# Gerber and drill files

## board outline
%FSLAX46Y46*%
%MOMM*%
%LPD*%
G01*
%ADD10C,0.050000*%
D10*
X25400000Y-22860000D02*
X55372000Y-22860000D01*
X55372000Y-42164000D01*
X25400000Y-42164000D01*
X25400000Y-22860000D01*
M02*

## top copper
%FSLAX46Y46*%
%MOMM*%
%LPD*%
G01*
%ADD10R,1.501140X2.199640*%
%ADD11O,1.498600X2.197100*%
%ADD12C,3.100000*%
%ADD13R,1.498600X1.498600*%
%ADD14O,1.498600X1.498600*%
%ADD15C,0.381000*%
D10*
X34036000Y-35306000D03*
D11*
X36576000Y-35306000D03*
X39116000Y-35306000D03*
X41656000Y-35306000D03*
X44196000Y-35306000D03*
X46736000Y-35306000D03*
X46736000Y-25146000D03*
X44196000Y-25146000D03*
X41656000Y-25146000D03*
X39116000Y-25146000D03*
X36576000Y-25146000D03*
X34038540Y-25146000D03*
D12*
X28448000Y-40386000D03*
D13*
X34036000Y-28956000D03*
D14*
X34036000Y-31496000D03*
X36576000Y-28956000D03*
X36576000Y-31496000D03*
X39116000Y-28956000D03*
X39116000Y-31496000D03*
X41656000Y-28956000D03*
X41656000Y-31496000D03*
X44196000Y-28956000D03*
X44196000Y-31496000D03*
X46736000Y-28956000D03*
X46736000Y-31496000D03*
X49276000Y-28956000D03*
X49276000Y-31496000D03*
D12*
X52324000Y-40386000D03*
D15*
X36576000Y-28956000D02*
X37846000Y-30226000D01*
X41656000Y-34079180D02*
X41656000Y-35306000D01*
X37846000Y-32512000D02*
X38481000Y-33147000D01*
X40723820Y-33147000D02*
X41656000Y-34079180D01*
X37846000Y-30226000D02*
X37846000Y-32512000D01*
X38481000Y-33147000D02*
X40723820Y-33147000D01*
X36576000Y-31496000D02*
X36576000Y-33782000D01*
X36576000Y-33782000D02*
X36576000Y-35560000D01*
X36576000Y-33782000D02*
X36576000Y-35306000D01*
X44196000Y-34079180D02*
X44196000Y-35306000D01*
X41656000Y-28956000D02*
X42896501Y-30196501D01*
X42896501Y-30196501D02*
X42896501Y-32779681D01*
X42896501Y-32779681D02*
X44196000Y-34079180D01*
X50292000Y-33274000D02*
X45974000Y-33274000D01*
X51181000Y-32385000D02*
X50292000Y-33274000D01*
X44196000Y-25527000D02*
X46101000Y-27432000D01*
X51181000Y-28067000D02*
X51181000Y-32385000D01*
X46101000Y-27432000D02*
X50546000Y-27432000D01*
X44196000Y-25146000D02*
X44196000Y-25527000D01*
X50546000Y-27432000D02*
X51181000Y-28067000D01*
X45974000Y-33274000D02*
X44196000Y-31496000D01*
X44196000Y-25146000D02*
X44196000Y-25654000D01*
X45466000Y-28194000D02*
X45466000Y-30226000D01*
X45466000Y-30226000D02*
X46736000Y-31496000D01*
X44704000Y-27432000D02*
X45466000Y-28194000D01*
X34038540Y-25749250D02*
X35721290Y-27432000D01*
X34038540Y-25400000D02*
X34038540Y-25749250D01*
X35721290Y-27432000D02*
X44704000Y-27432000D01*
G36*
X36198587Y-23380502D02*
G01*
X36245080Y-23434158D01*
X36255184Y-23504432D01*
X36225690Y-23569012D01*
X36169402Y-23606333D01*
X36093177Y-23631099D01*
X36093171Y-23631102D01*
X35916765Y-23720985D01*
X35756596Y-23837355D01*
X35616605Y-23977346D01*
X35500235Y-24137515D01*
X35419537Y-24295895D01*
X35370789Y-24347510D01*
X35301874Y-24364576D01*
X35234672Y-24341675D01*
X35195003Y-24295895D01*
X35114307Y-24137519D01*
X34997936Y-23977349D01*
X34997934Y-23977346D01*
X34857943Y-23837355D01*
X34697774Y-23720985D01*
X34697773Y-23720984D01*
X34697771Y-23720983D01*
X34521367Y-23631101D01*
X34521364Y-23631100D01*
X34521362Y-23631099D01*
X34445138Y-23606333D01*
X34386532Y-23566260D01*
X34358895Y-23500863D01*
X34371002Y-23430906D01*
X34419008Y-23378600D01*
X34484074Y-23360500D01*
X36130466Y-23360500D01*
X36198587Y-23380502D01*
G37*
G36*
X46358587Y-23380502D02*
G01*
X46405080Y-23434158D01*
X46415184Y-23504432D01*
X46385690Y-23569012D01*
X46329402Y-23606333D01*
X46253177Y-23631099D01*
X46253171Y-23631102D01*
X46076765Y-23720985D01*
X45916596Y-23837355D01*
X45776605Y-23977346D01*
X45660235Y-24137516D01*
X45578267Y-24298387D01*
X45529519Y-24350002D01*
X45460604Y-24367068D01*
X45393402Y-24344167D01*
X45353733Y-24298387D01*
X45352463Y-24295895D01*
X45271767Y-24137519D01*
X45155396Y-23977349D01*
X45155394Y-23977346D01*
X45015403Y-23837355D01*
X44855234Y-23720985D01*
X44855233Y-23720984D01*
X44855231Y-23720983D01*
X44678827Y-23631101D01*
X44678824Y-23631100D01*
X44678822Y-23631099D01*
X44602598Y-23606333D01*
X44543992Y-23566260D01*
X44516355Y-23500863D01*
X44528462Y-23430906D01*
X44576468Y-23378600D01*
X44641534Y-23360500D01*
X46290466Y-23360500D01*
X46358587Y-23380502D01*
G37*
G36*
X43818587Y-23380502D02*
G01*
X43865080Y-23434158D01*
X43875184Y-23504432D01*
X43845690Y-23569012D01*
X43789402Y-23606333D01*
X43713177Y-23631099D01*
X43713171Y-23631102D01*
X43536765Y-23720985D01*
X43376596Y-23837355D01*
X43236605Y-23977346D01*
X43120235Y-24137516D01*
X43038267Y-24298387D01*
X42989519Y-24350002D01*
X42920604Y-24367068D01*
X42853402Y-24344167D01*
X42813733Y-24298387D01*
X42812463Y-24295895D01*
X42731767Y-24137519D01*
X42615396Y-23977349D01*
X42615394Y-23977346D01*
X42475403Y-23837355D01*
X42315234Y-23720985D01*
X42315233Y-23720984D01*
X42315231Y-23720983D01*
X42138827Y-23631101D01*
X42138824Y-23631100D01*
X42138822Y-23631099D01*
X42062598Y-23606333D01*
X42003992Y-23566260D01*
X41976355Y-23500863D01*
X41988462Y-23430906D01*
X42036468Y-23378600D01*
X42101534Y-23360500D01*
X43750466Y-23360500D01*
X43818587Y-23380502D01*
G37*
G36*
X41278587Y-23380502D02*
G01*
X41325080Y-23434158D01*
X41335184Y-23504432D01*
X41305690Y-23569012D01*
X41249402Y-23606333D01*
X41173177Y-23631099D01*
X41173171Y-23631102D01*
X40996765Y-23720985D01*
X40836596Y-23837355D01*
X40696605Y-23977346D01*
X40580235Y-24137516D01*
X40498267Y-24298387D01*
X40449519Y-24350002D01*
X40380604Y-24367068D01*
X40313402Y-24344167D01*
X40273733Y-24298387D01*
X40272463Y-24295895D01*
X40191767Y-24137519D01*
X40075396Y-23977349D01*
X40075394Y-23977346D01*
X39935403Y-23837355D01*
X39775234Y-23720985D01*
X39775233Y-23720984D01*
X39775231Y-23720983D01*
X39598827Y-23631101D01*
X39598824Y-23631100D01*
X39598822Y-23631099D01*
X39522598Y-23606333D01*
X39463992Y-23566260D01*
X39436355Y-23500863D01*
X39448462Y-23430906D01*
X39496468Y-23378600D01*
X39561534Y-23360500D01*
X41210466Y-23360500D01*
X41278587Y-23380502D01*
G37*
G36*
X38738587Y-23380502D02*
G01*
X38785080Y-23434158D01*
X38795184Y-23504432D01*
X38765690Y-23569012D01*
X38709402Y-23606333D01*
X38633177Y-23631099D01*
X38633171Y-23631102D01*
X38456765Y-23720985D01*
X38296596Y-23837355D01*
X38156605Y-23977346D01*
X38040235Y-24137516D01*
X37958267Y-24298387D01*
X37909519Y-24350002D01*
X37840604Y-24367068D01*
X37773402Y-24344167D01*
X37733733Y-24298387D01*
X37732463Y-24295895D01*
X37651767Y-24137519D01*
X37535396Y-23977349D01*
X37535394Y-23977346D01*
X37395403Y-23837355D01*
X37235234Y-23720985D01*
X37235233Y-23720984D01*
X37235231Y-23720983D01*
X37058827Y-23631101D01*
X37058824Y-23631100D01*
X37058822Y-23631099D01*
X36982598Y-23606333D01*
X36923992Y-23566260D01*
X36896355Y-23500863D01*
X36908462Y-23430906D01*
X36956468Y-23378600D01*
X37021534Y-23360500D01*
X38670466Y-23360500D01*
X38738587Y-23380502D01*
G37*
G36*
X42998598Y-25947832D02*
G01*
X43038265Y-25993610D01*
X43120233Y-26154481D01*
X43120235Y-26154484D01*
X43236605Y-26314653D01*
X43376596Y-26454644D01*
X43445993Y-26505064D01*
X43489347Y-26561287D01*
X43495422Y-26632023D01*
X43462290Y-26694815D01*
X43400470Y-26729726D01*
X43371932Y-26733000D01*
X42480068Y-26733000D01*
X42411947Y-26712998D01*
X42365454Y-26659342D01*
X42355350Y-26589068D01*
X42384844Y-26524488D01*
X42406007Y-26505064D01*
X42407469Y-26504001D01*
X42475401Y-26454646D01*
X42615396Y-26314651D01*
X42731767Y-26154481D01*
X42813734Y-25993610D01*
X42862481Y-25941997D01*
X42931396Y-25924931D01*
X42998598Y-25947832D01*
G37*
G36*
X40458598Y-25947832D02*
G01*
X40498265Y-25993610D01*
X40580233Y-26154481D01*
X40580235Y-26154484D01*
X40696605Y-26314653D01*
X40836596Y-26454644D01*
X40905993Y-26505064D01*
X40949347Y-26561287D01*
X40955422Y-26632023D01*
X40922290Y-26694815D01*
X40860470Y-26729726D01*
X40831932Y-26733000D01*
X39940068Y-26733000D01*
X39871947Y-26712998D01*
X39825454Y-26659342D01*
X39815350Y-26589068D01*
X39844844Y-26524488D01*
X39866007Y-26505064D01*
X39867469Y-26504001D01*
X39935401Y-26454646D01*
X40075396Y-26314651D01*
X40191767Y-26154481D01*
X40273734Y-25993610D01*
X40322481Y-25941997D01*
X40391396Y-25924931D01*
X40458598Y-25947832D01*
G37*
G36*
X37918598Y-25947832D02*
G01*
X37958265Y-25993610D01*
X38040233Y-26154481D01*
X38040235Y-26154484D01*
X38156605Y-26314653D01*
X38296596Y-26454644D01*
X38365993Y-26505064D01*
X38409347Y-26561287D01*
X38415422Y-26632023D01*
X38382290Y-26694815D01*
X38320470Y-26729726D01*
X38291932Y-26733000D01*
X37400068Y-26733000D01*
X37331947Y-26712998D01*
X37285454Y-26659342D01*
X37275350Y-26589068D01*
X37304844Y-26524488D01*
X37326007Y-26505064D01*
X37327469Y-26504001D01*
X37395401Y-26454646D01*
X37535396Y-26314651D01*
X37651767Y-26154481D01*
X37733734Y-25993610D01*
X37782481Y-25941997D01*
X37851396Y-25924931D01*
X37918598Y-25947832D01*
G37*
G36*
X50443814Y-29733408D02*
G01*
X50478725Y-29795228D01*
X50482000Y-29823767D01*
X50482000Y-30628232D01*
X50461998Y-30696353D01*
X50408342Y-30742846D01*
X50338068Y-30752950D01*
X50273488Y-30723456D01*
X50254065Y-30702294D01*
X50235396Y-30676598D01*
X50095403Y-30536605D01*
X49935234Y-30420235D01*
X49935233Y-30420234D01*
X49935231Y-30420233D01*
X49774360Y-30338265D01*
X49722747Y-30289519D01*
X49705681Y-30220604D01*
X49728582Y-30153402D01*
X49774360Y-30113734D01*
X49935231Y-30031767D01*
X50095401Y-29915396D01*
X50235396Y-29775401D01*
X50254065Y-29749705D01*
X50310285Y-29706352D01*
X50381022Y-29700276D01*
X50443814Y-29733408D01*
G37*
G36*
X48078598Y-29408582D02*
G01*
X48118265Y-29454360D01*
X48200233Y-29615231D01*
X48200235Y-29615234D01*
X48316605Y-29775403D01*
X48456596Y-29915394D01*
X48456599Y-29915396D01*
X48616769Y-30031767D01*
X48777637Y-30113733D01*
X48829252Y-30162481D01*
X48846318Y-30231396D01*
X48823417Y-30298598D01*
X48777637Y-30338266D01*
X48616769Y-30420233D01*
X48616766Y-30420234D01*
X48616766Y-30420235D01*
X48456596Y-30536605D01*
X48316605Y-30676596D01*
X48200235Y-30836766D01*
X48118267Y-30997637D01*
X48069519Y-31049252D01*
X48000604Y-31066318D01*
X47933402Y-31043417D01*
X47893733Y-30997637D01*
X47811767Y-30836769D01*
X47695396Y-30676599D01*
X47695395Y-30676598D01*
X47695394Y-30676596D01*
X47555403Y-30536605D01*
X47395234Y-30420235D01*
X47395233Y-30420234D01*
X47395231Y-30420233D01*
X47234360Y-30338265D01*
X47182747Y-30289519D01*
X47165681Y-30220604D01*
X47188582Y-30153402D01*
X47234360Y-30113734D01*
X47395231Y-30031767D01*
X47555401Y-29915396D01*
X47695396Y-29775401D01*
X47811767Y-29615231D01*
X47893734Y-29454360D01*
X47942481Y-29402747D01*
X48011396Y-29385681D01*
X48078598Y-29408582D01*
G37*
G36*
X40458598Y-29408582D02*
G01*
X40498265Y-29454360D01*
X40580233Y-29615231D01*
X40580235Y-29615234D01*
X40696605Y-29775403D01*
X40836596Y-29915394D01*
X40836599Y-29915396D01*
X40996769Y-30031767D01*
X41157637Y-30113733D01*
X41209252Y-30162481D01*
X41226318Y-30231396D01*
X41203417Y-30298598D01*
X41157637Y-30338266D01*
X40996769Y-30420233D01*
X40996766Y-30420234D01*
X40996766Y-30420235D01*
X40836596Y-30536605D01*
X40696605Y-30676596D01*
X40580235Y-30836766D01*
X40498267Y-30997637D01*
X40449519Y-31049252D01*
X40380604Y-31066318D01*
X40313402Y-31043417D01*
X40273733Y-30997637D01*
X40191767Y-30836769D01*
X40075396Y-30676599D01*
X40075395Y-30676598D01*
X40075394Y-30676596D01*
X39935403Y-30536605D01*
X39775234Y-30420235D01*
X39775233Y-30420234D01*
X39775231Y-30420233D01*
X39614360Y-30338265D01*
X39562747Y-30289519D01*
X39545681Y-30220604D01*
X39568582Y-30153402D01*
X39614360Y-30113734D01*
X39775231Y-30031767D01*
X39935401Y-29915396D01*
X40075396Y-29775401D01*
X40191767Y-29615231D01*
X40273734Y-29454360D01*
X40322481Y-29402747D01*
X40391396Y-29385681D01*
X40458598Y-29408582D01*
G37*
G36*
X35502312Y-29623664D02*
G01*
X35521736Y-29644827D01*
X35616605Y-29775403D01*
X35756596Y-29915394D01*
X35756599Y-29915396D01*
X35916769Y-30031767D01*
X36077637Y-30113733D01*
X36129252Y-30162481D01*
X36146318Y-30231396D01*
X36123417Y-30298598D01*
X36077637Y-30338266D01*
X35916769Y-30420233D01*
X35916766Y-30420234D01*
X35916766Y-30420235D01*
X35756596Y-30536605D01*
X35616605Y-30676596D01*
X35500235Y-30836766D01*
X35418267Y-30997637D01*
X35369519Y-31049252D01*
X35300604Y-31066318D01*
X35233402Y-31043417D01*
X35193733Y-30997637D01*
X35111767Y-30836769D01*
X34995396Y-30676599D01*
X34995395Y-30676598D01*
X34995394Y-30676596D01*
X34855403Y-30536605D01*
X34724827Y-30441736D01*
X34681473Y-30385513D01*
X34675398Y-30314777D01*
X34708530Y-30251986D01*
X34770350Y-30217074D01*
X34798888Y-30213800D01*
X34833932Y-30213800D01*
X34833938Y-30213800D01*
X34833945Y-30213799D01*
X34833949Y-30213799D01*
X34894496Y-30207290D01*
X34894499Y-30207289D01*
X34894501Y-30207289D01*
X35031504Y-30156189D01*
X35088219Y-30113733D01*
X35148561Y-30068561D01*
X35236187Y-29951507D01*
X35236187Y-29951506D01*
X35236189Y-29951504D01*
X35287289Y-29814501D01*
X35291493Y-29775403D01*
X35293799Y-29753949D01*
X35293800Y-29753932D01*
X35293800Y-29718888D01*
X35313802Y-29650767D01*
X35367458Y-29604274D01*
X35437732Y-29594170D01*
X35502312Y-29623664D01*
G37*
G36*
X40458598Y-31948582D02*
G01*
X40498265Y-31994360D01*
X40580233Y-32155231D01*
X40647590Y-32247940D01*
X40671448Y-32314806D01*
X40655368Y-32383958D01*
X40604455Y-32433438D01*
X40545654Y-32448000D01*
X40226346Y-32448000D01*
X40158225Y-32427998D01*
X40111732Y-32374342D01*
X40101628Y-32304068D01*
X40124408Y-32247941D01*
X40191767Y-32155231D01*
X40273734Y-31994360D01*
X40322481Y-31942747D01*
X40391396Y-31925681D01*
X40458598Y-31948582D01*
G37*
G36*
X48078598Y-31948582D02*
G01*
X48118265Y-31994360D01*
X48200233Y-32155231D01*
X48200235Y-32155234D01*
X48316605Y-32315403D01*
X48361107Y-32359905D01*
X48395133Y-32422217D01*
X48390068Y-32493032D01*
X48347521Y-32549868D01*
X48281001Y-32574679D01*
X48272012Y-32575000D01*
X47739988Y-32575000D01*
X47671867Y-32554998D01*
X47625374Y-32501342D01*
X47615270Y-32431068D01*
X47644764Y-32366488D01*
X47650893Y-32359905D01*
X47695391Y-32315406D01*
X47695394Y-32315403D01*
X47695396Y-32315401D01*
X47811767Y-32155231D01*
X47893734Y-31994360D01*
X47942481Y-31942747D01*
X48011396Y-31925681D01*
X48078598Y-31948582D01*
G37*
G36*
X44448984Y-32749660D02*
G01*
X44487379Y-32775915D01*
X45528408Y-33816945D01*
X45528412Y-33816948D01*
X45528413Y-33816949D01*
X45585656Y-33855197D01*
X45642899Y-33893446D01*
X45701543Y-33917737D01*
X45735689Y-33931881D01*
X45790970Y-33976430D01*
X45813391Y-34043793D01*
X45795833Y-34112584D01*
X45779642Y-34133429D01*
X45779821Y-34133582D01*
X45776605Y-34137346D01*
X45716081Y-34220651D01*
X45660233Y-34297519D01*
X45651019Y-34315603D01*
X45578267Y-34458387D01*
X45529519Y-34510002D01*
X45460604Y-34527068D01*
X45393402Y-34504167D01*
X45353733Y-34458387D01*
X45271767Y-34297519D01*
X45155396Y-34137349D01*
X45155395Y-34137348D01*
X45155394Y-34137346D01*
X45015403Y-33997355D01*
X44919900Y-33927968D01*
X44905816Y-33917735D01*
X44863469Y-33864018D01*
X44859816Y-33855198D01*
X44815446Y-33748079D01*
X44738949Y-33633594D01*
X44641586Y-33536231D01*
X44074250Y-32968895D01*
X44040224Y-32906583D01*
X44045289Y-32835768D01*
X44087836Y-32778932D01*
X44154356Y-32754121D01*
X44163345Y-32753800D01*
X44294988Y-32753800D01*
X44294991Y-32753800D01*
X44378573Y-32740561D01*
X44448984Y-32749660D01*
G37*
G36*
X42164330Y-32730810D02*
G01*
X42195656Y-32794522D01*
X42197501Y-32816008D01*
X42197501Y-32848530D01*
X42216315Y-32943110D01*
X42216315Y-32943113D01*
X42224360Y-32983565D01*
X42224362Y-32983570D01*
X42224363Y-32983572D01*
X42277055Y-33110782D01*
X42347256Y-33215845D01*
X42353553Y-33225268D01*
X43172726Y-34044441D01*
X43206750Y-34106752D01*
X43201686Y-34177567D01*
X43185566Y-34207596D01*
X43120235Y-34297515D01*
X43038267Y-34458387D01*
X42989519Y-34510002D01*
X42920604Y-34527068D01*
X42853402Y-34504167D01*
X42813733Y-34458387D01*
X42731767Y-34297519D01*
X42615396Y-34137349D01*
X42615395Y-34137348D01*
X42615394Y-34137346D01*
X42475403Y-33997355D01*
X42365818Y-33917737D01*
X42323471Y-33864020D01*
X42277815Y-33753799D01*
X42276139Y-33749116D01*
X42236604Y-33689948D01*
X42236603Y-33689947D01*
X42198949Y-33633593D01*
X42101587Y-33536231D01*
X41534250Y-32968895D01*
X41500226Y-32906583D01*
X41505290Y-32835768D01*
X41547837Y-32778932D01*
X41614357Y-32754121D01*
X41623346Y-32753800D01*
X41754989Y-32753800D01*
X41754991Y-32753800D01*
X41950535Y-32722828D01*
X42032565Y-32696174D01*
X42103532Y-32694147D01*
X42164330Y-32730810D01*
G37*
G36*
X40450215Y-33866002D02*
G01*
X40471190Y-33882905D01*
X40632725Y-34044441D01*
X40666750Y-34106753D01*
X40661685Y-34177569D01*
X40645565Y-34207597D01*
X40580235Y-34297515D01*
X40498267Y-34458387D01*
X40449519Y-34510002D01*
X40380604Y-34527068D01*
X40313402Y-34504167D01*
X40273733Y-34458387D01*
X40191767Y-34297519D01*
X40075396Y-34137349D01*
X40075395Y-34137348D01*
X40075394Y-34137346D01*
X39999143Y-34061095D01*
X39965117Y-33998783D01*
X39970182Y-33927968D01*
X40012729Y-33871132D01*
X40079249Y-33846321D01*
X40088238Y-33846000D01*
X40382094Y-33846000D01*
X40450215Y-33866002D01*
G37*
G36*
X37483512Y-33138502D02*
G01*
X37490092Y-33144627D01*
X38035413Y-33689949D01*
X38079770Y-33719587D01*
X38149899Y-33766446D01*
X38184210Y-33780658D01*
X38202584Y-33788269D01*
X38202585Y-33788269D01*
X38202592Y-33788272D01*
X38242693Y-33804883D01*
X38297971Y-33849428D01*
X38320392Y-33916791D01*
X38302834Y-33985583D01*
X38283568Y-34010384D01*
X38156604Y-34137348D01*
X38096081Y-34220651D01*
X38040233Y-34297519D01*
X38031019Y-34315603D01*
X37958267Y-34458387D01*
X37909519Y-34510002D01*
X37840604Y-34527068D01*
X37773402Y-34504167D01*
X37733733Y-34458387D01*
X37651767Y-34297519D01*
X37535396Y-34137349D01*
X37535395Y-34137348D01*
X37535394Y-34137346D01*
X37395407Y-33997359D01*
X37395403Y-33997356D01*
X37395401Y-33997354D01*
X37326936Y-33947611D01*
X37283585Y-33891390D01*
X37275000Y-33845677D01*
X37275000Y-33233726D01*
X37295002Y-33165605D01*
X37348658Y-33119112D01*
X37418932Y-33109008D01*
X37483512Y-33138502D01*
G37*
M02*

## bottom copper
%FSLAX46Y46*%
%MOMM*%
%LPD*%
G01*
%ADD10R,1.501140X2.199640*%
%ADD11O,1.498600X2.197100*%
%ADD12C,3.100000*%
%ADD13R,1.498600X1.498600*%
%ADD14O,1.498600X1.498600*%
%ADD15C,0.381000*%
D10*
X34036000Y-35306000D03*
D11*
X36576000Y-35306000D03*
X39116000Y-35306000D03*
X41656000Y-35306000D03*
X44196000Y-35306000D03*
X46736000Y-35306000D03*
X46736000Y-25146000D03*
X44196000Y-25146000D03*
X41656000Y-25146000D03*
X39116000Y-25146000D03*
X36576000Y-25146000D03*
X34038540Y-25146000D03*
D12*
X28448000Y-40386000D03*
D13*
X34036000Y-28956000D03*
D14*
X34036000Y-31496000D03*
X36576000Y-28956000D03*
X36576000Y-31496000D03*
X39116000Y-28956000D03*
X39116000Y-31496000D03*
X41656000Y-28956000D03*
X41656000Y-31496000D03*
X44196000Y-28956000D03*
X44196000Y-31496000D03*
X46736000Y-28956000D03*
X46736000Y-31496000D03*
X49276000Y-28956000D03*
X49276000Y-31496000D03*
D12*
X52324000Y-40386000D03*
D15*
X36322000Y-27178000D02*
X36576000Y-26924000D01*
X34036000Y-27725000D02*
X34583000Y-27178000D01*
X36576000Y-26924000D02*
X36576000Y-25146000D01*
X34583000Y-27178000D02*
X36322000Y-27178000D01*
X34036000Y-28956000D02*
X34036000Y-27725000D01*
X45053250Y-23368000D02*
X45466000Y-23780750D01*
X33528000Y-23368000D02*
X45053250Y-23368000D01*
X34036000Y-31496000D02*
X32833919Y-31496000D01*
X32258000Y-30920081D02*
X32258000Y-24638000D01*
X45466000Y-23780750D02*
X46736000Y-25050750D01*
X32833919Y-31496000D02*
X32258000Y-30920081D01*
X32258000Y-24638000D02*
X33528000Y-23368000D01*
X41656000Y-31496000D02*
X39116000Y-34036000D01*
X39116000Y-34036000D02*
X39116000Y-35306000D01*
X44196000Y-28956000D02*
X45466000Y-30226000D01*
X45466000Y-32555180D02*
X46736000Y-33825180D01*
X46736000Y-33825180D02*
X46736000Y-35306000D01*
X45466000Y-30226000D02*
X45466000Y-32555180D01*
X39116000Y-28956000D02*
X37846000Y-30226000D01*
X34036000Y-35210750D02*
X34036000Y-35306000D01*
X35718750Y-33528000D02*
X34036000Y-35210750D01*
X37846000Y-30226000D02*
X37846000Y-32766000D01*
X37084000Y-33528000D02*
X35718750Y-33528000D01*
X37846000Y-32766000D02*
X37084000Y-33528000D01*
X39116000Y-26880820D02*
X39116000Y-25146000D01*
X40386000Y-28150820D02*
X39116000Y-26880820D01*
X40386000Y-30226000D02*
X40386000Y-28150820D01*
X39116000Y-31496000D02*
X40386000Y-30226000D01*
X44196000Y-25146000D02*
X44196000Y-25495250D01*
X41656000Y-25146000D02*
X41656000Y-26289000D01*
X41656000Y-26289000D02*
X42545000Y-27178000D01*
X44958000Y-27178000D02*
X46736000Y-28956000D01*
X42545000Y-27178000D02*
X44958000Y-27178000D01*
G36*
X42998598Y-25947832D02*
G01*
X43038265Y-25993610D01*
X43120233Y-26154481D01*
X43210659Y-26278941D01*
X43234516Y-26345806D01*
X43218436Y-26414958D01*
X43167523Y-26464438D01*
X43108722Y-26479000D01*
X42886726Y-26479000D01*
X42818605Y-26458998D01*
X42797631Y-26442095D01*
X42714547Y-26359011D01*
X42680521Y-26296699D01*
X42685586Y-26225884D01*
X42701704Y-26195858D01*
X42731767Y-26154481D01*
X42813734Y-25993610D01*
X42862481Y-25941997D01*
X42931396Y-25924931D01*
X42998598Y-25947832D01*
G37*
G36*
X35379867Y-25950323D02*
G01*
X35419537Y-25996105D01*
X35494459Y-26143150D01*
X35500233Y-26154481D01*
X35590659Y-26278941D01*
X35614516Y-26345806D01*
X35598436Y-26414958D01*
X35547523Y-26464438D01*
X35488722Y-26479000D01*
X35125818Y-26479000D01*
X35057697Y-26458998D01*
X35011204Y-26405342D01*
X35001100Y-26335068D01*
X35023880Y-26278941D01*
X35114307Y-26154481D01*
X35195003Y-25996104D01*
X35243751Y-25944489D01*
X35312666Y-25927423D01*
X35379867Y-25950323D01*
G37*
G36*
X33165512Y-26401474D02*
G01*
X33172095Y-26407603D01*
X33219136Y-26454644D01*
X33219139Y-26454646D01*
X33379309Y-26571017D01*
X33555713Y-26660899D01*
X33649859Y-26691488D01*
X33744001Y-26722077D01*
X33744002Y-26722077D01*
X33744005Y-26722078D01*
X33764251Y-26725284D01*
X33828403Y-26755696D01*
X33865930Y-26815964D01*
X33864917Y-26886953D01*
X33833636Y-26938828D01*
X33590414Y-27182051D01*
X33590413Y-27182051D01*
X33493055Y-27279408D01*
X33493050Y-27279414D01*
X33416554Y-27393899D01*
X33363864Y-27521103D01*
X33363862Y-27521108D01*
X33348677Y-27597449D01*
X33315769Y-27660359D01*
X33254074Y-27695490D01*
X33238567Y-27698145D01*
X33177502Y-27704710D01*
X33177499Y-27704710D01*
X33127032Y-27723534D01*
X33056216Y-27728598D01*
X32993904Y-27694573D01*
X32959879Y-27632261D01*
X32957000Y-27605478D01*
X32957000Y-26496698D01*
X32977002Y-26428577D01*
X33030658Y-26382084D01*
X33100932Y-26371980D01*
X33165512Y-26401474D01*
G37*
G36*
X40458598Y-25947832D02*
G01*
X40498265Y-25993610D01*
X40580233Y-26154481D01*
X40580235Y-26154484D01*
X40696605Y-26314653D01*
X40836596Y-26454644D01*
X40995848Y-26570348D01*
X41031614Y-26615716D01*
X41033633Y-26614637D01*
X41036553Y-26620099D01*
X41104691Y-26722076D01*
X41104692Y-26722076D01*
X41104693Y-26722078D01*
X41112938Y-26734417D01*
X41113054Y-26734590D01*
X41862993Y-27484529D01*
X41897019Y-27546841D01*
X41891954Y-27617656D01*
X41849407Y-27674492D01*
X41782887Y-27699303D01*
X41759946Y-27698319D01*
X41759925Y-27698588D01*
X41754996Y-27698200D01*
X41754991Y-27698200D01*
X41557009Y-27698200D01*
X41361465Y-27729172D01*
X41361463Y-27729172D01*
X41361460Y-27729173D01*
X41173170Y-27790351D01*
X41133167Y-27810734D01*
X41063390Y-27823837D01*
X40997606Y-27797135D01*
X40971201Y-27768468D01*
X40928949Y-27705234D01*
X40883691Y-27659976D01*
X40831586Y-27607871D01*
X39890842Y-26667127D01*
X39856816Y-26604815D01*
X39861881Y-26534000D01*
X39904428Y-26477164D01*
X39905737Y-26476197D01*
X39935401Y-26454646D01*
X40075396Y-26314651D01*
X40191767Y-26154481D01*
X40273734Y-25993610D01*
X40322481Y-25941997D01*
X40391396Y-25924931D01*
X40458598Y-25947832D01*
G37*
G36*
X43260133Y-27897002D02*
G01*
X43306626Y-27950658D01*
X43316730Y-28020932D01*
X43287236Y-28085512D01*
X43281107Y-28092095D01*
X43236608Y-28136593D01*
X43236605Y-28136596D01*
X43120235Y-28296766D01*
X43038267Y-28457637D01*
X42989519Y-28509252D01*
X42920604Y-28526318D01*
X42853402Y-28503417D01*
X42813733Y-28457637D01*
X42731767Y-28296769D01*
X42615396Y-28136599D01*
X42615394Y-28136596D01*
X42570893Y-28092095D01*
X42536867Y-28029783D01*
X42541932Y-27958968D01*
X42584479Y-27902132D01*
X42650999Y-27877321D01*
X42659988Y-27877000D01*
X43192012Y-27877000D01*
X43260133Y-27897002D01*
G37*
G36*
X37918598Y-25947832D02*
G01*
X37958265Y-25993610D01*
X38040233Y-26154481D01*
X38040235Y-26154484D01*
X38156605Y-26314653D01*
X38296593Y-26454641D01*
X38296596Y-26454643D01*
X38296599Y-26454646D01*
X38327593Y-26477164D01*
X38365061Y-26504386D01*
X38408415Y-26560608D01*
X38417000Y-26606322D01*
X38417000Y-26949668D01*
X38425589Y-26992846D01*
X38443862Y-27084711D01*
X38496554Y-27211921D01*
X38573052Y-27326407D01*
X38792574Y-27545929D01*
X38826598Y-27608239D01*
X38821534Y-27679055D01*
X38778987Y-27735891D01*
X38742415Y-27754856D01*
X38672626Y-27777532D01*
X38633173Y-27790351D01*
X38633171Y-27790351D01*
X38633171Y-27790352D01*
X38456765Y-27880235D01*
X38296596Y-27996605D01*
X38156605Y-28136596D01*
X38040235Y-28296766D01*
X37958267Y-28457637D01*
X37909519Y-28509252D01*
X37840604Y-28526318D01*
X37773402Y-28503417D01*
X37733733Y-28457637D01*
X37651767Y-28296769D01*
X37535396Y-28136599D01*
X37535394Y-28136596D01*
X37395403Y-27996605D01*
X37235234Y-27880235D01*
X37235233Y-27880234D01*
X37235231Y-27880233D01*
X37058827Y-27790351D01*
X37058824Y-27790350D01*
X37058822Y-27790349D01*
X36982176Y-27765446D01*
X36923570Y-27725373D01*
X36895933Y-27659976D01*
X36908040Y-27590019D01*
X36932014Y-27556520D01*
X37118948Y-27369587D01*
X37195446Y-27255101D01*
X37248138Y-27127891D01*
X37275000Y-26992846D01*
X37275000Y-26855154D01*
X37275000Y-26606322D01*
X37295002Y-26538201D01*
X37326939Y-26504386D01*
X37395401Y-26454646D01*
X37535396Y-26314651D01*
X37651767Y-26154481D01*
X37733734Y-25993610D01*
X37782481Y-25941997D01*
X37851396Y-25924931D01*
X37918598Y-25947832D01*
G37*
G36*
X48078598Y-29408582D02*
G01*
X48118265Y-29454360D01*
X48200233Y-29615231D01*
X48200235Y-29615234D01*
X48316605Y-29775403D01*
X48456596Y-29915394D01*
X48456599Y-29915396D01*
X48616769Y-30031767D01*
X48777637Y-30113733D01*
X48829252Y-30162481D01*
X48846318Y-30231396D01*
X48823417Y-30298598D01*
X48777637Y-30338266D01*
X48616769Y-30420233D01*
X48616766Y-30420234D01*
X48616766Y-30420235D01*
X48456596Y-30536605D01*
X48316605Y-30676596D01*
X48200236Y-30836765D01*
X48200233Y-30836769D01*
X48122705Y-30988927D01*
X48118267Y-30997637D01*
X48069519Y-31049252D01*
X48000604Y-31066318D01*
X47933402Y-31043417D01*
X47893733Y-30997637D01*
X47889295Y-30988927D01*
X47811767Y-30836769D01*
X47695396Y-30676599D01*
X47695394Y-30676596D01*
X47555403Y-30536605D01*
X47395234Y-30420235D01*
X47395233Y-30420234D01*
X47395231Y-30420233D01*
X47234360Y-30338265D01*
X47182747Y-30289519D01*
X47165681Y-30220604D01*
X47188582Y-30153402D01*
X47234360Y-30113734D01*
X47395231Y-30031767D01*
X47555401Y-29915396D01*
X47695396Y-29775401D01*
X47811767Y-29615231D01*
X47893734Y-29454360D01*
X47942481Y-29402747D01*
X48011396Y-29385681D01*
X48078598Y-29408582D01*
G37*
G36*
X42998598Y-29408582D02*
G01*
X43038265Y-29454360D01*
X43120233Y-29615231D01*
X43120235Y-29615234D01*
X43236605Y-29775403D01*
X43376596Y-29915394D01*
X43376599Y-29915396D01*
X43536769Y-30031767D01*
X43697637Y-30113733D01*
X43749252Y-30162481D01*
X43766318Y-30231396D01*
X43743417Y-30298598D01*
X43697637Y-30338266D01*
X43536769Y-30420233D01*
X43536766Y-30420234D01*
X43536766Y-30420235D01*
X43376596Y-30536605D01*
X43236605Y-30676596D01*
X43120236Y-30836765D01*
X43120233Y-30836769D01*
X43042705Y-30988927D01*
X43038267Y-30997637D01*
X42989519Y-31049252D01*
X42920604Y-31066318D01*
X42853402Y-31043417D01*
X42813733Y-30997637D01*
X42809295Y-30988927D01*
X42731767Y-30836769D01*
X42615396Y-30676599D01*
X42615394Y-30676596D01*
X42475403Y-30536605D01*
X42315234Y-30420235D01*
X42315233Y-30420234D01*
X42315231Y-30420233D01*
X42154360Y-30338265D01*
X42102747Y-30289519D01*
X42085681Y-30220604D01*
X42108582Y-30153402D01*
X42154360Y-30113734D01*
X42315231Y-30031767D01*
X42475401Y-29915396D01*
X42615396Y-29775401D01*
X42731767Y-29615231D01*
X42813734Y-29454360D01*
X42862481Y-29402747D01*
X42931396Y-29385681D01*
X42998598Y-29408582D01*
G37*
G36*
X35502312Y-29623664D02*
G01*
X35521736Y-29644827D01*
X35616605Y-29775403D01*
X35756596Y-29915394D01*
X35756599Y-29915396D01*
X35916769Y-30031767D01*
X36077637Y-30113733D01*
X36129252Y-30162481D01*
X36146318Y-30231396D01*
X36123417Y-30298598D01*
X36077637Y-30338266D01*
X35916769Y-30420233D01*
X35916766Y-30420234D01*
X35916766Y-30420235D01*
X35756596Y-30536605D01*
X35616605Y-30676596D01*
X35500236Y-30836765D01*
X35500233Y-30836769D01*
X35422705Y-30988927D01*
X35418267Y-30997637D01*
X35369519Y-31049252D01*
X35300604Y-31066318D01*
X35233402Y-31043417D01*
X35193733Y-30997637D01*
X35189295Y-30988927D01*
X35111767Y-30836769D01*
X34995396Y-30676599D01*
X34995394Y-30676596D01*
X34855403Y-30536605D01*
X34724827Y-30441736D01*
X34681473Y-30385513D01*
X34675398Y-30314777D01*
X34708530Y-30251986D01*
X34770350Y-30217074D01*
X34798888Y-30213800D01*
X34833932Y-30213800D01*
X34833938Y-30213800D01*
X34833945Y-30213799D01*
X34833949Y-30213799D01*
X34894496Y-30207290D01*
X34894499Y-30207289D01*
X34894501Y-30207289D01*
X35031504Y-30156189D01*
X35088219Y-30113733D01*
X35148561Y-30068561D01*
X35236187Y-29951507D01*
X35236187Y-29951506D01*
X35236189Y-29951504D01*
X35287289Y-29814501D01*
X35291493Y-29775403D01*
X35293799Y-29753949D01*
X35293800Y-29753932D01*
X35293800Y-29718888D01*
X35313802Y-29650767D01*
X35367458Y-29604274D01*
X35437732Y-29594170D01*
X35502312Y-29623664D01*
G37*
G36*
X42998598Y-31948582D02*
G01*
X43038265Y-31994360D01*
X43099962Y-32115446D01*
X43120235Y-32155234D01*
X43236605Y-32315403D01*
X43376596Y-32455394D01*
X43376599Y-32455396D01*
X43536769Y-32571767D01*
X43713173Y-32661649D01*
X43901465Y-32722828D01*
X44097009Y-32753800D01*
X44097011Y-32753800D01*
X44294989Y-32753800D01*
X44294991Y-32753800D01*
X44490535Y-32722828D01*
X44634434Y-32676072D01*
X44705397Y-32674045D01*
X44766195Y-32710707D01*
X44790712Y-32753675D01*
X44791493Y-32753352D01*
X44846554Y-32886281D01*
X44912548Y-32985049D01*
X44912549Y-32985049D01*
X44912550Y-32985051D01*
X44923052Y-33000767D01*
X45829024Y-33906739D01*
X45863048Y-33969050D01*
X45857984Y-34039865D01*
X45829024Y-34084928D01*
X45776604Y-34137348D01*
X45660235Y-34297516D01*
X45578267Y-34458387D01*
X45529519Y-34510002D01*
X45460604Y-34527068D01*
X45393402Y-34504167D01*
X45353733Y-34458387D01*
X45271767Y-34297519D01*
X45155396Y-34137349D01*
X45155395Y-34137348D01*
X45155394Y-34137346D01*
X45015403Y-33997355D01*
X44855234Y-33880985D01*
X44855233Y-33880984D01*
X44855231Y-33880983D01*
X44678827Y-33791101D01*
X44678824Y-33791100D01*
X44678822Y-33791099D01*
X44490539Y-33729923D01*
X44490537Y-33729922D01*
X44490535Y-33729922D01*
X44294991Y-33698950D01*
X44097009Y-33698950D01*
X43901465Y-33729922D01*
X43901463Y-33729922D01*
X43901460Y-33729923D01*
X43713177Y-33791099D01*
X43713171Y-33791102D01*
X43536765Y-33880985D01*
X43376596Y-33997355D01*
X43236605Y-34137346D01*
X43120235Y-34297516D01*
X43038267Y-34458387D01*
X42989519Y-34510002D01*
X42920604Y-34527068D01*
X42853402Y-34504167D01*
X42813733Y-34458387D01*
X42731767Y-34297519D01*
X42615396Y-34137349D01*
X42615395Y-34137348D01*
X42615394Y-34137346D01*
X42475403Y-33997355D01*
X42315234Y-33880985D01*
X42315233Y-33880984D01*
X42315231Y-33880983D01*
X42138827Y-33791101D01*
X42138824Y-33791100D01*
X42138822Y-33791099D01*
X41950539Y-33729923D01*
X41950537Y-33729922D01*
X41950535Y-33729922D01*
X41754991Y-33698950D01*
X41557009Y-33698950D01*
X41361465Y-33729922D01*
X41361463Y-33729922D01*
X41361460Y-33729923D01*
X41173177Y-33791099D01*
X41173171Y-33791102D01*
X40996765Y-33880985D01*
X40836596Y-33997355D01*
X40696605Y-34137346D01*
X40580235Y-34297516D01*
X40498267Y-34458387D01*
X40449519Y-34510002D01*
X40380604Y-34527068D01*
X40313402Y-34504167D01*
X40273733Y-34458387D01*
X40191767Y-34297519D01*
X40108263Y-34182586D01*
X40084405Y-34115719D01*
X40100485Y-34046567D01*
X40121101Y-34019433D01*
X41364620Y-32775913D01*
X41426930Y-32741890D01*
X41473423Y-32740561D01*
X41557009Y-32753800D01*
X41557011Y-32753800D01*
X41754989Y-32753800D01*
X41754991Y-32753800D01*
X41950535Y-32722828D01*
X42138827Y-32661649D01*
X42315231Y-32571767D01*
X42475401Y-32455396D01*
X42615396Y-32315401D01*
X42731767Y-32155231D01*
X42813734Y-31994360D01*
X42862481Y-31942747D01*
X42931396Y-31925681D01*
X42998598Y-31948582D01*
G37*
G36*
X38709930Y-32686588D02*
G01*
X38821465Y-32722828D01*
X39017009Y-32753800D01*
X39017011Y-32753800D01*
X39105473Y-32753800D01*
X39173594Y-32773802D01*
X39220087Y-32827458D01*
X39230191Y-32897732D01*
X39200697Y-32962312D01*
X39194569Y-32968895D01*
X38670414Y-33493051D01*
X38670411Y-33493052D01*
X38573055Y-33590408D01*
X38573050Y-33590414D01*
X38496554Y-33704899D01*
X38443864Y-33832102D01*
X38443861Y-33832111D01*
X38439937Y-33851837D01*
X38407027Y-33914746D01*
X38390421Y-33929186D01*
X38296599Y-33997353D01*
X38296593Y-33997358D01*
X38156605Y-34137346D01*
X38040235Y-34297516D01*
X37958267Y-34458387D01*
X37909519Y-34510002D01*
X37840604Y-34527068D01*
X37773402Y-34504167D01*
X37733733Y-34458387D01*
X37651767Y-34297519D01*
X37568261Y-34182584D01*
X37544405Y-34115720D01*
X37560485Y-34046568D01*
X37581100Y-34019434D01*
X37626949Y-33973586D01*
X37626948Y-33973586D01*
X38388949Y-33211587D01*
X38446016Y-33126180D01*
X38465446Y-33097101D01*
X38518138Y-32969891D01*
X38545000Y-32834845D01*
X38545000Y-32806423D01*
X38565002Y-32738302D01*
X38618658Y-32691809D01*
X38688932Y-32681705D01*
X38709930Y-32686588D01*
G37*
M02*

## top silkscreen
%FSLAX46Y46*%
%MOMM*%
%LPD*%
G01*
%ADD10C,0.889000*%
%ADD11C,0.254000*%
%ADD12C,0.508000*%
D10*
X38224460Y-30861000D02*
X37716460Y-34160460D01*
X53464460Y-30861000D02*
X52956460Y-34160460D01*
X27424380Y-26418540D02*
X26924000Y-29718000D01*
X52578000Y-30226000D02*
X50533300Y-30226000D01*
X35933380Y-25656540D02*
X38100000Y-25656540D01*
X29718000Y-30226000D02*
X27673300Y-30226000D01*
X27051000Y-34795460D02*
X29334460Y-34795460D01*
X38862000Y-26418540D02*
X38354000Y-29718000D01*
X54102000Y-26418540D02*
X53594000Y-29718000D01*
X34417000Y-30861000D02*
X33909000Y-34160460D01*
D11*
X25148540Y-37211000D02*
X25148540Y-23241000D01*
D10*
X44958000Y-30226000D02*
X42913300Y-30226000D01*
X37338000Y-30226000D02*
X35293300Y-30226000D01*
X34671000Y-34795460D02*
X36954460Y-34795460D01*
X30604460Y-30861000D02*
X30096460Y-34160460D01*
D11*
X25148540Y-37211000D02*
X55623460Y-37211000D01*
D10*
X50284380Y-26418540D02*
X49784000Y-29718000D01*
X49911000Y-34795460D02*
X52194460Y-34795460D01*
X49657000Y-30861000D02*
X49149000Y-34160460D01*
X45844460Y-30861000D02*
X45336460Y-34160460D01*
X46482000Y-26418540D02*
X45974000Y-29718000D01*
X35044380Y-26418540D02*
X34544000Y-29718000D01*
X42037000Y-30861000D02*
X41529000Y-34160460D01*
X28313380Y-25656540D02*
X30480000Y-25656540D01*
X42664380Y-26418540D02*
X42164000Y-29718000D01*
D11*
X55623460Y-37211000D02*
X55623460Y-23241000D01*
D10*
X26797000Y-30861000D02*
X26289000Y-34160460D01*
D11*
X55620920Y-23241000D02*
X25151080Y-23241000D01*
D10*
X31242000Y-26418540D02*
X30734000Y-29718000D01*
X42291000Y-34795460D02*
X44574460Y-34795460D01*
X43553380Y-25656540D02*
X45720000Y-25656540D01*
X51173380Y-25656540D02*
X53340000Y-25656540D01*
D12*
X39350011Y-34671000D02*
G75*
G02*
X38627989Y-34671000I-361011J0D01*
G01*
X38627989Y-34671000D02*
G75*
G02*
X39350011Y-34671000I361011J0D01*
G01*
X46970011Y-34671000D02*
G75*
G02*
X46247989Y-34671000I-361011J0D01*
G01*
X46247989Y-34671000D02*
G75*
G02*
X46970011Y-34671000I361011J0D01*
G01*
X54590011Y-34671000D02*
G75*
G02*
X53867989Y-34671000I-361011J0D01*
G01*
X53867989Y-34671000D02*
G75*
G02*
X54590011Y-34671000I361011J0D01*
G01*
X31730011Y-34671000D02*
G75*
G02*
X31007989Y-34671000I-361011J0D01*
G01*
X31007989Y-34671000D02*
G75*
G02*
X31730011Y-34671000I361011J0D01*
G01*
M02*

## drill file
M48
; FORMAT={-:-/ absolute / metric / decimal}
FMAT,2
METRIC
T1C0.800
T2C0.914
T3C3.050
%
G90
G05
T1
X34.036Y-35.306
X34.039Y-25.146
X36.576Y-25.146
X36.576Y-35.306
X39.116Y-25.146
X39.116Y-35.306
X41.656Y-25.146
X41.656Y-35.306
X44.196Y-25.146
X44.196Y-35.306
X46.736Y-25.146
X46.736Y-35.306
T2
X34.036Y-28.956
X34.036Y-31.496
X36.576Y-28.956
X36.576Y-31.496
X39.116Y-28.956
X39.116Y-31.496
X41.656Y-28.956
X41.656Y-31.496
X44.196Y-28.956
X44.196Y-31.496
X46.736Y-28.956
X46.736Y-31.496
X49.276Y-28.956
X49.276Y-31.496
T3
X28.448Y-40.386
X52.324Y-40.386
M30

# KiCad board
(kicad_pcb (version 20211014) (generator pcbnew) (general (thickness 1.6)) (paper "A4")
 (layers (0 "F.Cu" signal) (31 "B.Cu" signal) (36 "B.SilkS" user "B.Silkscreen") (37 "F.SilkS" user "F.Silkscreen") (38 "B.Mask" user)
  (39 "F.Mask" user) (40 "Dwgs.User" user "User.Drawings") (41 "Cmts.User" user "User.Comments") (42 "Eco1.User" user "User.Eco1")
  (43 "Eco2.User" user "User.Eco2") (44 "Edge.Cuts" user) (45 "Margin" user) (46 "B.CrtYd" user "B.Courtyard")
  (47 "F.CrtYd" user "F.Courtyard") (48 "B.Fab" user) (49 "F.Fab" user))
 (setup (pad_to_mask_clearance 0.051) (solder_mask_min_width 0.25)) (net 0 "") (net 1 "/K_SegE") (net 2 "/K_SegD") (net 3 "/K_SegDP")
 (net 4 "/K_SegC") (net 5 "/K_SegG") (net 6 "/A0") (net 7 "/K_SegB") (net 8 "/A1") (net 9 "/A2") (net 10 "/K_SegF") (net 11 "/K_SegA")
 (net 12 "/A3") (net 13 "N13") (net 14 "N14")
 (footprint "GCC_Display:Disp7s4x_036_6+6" (layer "F.Cu") (at 40.386 30.226)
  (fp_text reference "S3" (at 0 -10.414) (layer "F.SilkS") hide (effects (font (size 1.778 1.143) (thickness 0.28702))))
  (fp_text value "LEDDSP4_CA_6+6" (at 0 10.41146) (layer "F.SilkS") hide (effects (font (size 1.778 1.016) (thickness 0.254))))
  (fp_line (start -2.16154 0.635) (end -2.66954 3.93446) (layer "F.SilkS") (width 0.889))
  (fp_line (start 13.07846 0.635) (end 12.57046 3.93446) (layer "F.SilkS") (width 0.889))
  (fp_line (start -12.96162 -3.80746) (end -13.462 -0.508) (layer "F.SilkS") (width 0.889))
  (fp_line (start 12.192 0) (end 10.1473 0) (layer "F.SilkS") (width 0.889))
  (fp_line (start -4.45262 -4.56946) (end -2.286 -4.56946) (layer "F.SilkS") (width 0.889))
  (fp_line (start -10.668 0) (end -12.7127 0) (layer "F.SilkS") (width 0.889))
  (fp_line (start -13.335 4.56946) (end -11.05154 4.56946) (layer "F.SilkS") (width 0.889))
  (fp_line (start -1.524 -3.80746) (end -2.032 -0.508) (layer "F.SilkS") (width 0.889))
  (fp_line (start 13.716 -3.80746) (end 13.208 -0.508) (layer "F.SilkS") (width 0.889))
  (fp_line (start -5.969 0.635) (end -6.477 3.93446) (layer "F.SilkS") (width 0.889))
  (fp_line (start -15.23746 6.985) (end -15.23746 -6.985) (layer "F.SilkS") (width 0.254))
  (fp_line (start 4.572 0) (end 2.5273 0) (layer "F.SilkS") (width 0.889))
  (fp_line (start -3.048 0) (end -5.0927 0) (layer "F.SilkS") (width 0.889))
  (fp_line (start -5.715 4.56946) (end -3.43154 4.56946) (layer "F.SilkS") (width 0.889))
  (fp_line (start -9.78154 0.635) (end -10.28954 3.93446) (layer "F.SilkS") (width 0.889))
  (fp_line (start -15.23746 6.985) (end 15.23746 6.985) (layer "F.SilkS") (width 0.254))
  (fp_line (start 9.89838 -3.80746) (end 9.398 -0.508) (layer "F.SilkS") (width 0.889))
  (fp_line (start 9.525 4.56946) (end 11.80846 4.56946) (layer "F.SilkS") (width 0.889))
  (fp_line (start 9.271 0.635) (end 8.763 3.93446) (layer "F.SilkS") (width 0.889))
  (fp_line (start 5.45846 0.635) (end 4.95046 3.93446) (layer "F.SilkS") (width 0.889))
  (fp_line (start 6.096 -3.80746) (end 5.588 -0.508) (layer "F.SilkS") (width 0.889))
  (fp_line (start -5.34162 -3.80746) (end -5.842 -0.508) (layer "F.SilkS") (width 0.889))
  (fp_line (start 1.651 0.635) (end 1.143 3.93446) (layer "F.SilkS") (width 0.889))
  (fp_line (start -12.07262 -4.56946) (end -9.906 -4.56946) (layer "F.SilkS") (width 0.889))
  (fp_line (start 2.27838 -3.80746) (end 1.778 -0.508) (layer "F.SilkS") (width 0.889))
  (fp_line (start 15.23746 6.985) (end 15.23746 -6.985) (layer "F.SilkS") (width 0.254))
  (fp_line (start -13.589 0.635) (end -14.097 3.93446) (layer "F.SilkS") (width 0.889))
  (fp_line (start 15.23492 -6.985) (end -15.23492 -6.985) (layer "F.SilkS") (width 0.254))
  (fp_line (start -9.144 -3.80746) (end -9.652 -0.508) (layer "F.SilkS") (width 0.889))
  (fp_line (start 1.905 4.56946) (end 4.18846 4.56946) (layer "F.SilkS") (width 0.889))
  (fp_line (start 3.16738 -4.56946) (end 5.334 -4.56946) (layer "F.SilkS") (width 0.889))
  (fp_line (start 10.78738 -4.56946) (end 12.954 -4.56946) (layer "F.SilkS") (width 0.889))
  (fp_circle (center -1.397 4.445) (end -1.143 4.18846) (layer "F.SilkS") (width 0.508) (fill none))
  (fp_circle (center 6.223 4.445) (end 6.477 4.18846) (layer "F.SilkS") (width 0.508) (fill none))
  (fp_circle (center 13.843 4.445) (end 14.097 4.18846) (layer "F.SilkS") (width 0.508) (fill none))
  (fp_circle (center -9.017 4.445) (end -8.763 4.18846) (layer "F.SilkS") (width 0.508) (fill none))
  (pad "1" thru_hole rect locked (at -6.35 5.08 90) (size 2.19964 1.50114) (drill 0.8001) (layers *.Cu *.Mask) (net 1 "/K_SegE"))
  (pad "2" thru_hole oval locked (at -3.81 5.08 90) (size 2.1971 1.4986) (drill 0.8001) (layers *.Cu *.Mask) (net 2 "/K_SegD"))
  (pad "3" thru_hole oval locked (at -1.27 5.08 90) (size 2.1971 1.4986) (drill 0.8001) (layers *.Cu *.Mask) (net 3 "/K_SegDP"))
  (pad "4" thru_hole oval locked (at 1.27 5.08 90) (size 2.1971 1.4986) (drill 0.8001) (layers *.Cu *.Mask) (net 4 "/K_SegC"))
  (pad "5" thru_hole oval locked (at 3.81 5.08 90) (size 2.1971 1.4986) (drill 0.8001) (layers *.Cu *.Mask) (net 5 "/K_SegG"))
  (pad "6" thru_hole oval locked (at 6.35 5.08 90) (size 2.1971 1.4986) (drill 0.8001) (layers *.Cu *.Mask) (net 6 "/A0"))
  (pad "7" thru_hole oval locked (at 6.35 -5.08 90) (size 2.1971 1.4986) (drill 0.8001) (layers *.Cu *.Mask) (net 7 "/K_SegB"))
  (pad "8" thru_hole oval locked (at 3.81 -5.08 90) (size 2.1971 1.4986) (drill 0.8001) (layers *.Cu *.Mask) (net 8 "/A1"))
  (pad "9" thru_hole oval locked (at 1.27 -5.08 90) (size 2.1971 1.4986) (drill 0.8001) (layers *.Cu *.Mask) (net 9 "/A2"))
  (pad "10" thru_hole oval locked (at -1.27 -5.08 90) (size 2.1971 1.4986) (drill 0.8001) (layers *.Cu *.Mask) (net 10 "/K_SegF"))
  (pad "11" thru_hole oval locked (at -3.81 -5.08 90) (size 2.1971 1.4986) (drill 0.8001) (layers *.Cu *.Mask) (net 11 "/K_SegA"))
  (pad "12" thru_hole oval locked (at -6.34746 -5.08 90) (size 2.1971 1.4986) (drill 0.8001) (layers *.Cu *.Mask) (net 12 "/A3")))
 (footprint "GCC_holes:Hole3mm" (layer "B.Cu") (at 28.448 40.386)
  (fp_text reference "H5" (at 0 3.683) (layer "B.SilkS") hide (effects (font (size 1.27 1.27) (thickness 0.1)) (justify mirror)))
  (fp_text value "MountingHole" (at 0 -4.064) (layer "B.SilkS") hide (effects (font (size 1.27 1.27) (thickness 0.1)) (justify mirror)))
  (pad "1" thru_hole circle locked (at 0 0) (size 3.1 3.1) (drill 3.05) (layers *.Cu *.Mask)))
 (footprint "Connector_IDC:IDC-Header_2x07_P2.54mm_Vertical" (layer "B.Cu") (at 34.036 28.956 -90)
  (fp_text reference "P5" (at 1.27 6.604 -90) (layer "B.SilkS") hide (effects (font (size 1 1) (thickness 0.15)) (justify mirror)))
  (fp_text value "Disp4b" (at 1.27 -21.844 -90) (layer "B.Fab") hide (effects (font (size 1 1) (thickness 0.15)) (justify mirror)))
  (pad "1" thru_hole rect locked (at 0 0 270) (size 1.4986 1.4986) (drill 0.9144) (layers *.Cu *.Mask) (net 11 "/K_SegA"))
  (pad "2" thru_hole oval locked (at 2.54 0 270) (size 1.4986 1.4986) (drill 0.9144) (layers *.Cu *.Mask) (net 7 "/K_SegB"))
  (pad "3" thru_hole oval locked (at 0 -2.54 270) (size 1.4986 1.4986) (drill 0.9144) (layers *.Cu *.Mask) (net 4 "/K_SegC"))
  (pad "4" thru_hole oval locked (at 2.54 -2.54 270) (size 1.4986 1.4986) (drill 0.9144) (layers *.Cu *.Mask) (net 2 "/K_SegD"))
  (pad "5" thru_hole oval locked (at 0 -5.08 270) (size 1.4986 1.4986) (drill 0.9144) (layers *.Cu *.Mask) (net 1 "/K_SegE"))
  (pad "6" thru_hole oval locked (at 2.54 -5.08 270) (size 1.4986 1.4986) (drill 0.9144) (layers *.Cu *.Mask) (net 10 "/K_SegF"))
  (pad "7" thru_hole oval locked (at 0 -7.62 270) (size 1.4986 1.4986) (drill 0.9144) (layers *.Cu *.Mask) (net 5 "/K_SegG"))
  (pad "8" thru_hole oval locked (at 2.54 -7.62 270) (size 1.4986 1.4986) (drill 0.9144) (layers *.Cu *.Mask) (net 3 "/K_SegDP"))
  (pad "9" thru_hole oval locked (at 0 -10.16 270) (size 1.4986 1.4986) (drill 0.9144) (layers *.Cu *.Mask) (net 6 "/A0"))
  (pad "10" thru_hole oval locked (at 2.54 -10.16 270) (size 1.4986 1.4986) (drill 0.9144) (layers *.Cu *.Mask) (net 8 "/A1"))
  (pad "11" thru_hole oval locked (at 0 -12.7 270) (size 1.4986 1.4986) (drill 0.9144) (layers *.Cu *.Mask) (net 9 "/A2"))
  (pad "12" thru_hole oval locked (at 2.54 -12.7 270) (size 1.4986 1.4986) (drill 0.9144) (layers *.Cu *.Mask) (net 12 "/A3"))
  (pad "13" thru_hole oval locked (at 0 -15.24 270) (size 1.4986 1.4986) (drill 0.9144) (layers *.Cu *.Mask) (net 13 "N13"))
  (pad "14" thru_hole oval locked (at 2.54 -15.24 270) (size 1.4986 1.4986) (drill 0.9144) (layers *.Cu *.Mask) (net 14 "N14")))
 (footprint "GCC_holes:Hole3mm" (layer "B.Cu") (at 52.324 40.386)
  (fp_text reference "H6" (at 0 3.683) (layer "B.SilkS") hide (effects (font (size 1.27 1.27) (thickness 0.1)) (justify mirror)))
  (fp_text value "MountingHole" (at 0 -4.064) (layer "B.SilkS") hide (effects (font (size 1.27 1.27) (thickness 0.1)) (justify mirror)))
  (pad "1" thru_hole circle locked (at 0 0) (size 3.1 3.1) (drill 3.05) (layers *.Cu *.Mask)))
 (gr_rect (start 25.4 22.86) (end 55.372 42.164) (layer "Edge.Cuts") (width 0.05) (fill none))
 (segment (start 36.322 27.178) (end 36.576 26.924) (width 0.381) (layer "B.Cu") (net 11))
 (segment (start 34.036 27.725) (end 34.583 27.178) (width 0.381) (layer "B.Cu") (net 11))
 (segment (start 36.576 26.924) (end 36.576 25.146) (width 0.381) (layer "B.Cu") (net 11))
 (segment (start 34.583 27.178) (end 36.322 27.178) (width 0.381) (layer "B.Cu") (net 11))
 (segment (start 34.036 28.956) (end 34.036 27.725) (width 0.381) (layer "B.Cu") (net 11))
 (segment (start 45.05325 23.368) (end 45.466 23.78075) (width 0.381) (layer "B.Cu") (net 7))
 (segment (start 33.528 23.368) (end 45.05325 23.368) (width 0.381) (layer "B.Cu") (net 7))
 (segment (start 34.036 31.496) (end 32.833919 31.496) (width 0.381) (layer "B.Cu") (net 7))
 (segment (start 32.258 30.920081) (end 32.258 24.638) (width 0.381) (layer "B.Cu") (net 7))
 (segment (start 45.466 23.78075) (end 46.736 25.05075) (width 0.381) (layer "B.Cu") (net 7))
 (segment (start 32.833919 31.496) (end 32.258 30.920081) (width 0.381) (layer "B.Cu") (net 7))
 (segment (start 32.258 24.638) (end 33.528 23.368) (width 0.381) (layer "B.Cu") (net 7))
 (segment (start 36.576 28.956) (end 37.846 30.226) (width 0.381) (layer "F.Cu") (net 4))
 (segment (start 41.656 34.07918) (end 41.656 35.306) (width 0.381) (layer "F.Cu") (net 4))
 (segment (start 37.846 32.512) (end 38.481 33.147) (width 0.381) (layer "F.Cu") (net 4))
 (segment (start 40.72382 33.147) (end 41.656 34.07918) (width 0.381) (layer "F.Cu") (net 4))
 (segment (start 37.846 30.226) (end 37.846 32.512) (width 0.381) (layer "F.Cu") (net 4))
 (segment (start 38.481 33.147) (end 40.72382 33.147) (width 0.381) (layer "F.Cu") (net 4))
 (segment (start 41.656 31.496) (end 39.116 34.036) (width 0.381) (layer "B.Cu") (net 3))
 (segment (start 39.116 34.036) (end 39.116 35.306) (width 0.381) (layer "B.Cu") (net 3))
 (segment (start 44.196 28.956) (end 45.466 30.226) (width 0.381) (layer "B.Cu") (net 6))
 (segment (start 45.466 32.55518) (end 46.736 33.82518) (width 0.381) (layer "B.Cu") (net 6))
 (segment (start 46.736 33.82518) (end 46.736 35.306) (width 0.381) (layer "B.Cu") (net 6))
 (segment (start 45.466 30.226) (end 45.466 32.55518) (width 0.381) (layer "B.Cu") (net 6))
 (segment (start 36.576 31.496) (end 36.576 33.782) (width 0.381) (layer "F.Cu") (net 2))
 (segment (start 36.576 33.782) (end 36.576 35.56) (width 0.381) (layer "F.Cu") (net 2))
 (segment (start 36.576 33.782) (end 36.576 35.306) (width 0.381) (layer "F.Cu") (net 2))
 (segment (start 39.116 28.956) (end 37.846 30.226) (width 0.381) (layer "B.Cu") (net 1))
 (segment (start 34.036 35.21075) (end 34.036 35.306) (width 0.381) (layer "B.Cu") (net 1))
 (segment (start 35.71875 33.528) (end 34.036 35.21075) (width 0.381) (layer "B.Cu") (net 1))
 (segment (start 37.846 30.226) (end 37.846 32.766) (width 0.381) (layer "B.Cu") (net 1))
 (segment (start 37.084 33.528) (end 35.71875 33.528) (width 0.381) (layer "B.Cu") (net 1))
 (segment (start 37.846 32.766) (end 37.084 33.528) (width 0.381) (layer "B.Cu") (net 1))
 (segment (start 44.196 34.07918) (end 44.196 35.306) (width 0.381) (layer "F.Cu") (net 5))
 (segment (start 41.656 28.956) (end 42.896501 30.196501) (width 0.381) (layer "F.Cu") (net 5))
 (segment (start 42.896501 30.196501) (end 42.896501 32.779681) (width 0.381) (layer "F.Cu") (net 5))
 (segment (start 42.896501 32.779681) (end 44.196 34.07918) (width 0.381) (layer "F.Cu") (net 5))
 (segment (start 39.116 26.88082) (end 39.116 25.146) (width 0.381) (layer "B.Cu") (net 10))
 (segment (start 40.386 28.15082) (end 39.116 26.88082) (width 0.381) (layer "B.Cu") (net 10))
 (segment (start 40.386 30.226) (end 40.386 28.15082) (width 0.381) (layer "B.Cu") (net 10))
 (segment (start 39.116 31.496) (end 40.386 30.226) (width 0.381) (layer "B.Cu") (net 10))
 (segment (start 50.292 33.274) (end 45.974 33.274) (width 0.381) (layer "F.Cu") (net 8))
 (segment (start 51.181 32.385) (end 50.292 33.274) (width 0.381) (layer "F.Cu") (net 8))
 (segment (start 44.196 25.527) (end 46.101 27.432) (width 0.381) (layer "F.Cu") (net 8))
 (segment (start 51.181 28.067) (end 51.181 32.385) (width 0.381) (layer "F.Cu") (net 8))
 (segment (start 46.101 27.432) (end 50.546 27.432) (width 0.381) (layer "F.Cu") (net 8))
 (segment (start 44.196 25.146) (end 44.196 25.527) (width 0.381) (layer "F.Cu") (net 8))
 (segment (start 50.546 27.432) (end 51.181 28.067) (width 0.381) (layer "F.Cu") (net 8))
 (segment (start 45.974 33.274) (end 44.196 31.496) (width 0.381) (layer "F.Cu") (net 8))
 (segment (start 44.196 25.146) (end 44.196 25.654) (width 0.381) (layer "F.Cu") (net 8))
 (segment (start 44.196 25.146) (end 44.196 25.49525) (width 0.381) (layer "B.Cu") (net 8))
 (segment (start 41.656 25.146) (end 41.656 26.289) (width 0.381) (layer "B.Cu") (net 9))
 (segment (start 41.656 26.289) (end 42.545 27.178) (width 0.381) (layer "B.Cu") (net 9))
 (segment (start 44.958 27.178) (end 46.736 28.956) (width 0.381) (layer "B.Cu") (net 9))
 (segment (start 42.545 27.178) (end 44.958 27.178) (width 0.381) (layer "B.Cu") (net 9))
 (segment (start 45.466 28.194) (end 45.466 30.226) (width 0.381) (layer "F.Cu") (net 12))
 (segment (start 45.466 30.226) (end 46.736 31.496) (width 0.381) (layer "F.Cu") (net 12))
 (segment (start 44.704 27.432) (end 45.466 28.194) (width 0.381) (layer "F.Cu") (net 12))
 (segment (start 34.03854 25.74925) (end 35.72129 27.432) (width 0.381) (layer "F.Cu") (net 12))
 (segment (start 34.03854 25.4) (end 34.03854 25.74925) (width 0.381) (layer "F.Cu") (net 12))
 (segment (start 35.72129 27.432) (end 44.704 27.432) (width 0.381) (layer "F.Cu") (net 12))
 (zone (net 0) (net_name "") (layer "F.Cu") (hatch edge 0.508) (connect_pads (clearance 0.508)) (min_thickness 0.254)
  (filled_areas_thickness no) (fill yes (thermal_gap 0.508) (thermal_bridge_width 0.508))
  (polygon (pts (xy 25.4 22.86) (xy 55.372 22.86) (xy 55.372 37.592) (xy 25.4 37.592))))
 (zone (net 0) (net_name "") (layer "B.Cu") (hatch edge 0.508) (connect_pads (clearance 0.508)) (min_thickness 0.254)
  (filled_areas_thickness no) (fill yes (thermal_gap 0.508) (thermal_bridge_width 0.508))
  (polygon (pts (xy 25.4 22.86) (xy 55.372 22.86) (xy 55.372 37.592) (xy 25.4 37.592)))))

